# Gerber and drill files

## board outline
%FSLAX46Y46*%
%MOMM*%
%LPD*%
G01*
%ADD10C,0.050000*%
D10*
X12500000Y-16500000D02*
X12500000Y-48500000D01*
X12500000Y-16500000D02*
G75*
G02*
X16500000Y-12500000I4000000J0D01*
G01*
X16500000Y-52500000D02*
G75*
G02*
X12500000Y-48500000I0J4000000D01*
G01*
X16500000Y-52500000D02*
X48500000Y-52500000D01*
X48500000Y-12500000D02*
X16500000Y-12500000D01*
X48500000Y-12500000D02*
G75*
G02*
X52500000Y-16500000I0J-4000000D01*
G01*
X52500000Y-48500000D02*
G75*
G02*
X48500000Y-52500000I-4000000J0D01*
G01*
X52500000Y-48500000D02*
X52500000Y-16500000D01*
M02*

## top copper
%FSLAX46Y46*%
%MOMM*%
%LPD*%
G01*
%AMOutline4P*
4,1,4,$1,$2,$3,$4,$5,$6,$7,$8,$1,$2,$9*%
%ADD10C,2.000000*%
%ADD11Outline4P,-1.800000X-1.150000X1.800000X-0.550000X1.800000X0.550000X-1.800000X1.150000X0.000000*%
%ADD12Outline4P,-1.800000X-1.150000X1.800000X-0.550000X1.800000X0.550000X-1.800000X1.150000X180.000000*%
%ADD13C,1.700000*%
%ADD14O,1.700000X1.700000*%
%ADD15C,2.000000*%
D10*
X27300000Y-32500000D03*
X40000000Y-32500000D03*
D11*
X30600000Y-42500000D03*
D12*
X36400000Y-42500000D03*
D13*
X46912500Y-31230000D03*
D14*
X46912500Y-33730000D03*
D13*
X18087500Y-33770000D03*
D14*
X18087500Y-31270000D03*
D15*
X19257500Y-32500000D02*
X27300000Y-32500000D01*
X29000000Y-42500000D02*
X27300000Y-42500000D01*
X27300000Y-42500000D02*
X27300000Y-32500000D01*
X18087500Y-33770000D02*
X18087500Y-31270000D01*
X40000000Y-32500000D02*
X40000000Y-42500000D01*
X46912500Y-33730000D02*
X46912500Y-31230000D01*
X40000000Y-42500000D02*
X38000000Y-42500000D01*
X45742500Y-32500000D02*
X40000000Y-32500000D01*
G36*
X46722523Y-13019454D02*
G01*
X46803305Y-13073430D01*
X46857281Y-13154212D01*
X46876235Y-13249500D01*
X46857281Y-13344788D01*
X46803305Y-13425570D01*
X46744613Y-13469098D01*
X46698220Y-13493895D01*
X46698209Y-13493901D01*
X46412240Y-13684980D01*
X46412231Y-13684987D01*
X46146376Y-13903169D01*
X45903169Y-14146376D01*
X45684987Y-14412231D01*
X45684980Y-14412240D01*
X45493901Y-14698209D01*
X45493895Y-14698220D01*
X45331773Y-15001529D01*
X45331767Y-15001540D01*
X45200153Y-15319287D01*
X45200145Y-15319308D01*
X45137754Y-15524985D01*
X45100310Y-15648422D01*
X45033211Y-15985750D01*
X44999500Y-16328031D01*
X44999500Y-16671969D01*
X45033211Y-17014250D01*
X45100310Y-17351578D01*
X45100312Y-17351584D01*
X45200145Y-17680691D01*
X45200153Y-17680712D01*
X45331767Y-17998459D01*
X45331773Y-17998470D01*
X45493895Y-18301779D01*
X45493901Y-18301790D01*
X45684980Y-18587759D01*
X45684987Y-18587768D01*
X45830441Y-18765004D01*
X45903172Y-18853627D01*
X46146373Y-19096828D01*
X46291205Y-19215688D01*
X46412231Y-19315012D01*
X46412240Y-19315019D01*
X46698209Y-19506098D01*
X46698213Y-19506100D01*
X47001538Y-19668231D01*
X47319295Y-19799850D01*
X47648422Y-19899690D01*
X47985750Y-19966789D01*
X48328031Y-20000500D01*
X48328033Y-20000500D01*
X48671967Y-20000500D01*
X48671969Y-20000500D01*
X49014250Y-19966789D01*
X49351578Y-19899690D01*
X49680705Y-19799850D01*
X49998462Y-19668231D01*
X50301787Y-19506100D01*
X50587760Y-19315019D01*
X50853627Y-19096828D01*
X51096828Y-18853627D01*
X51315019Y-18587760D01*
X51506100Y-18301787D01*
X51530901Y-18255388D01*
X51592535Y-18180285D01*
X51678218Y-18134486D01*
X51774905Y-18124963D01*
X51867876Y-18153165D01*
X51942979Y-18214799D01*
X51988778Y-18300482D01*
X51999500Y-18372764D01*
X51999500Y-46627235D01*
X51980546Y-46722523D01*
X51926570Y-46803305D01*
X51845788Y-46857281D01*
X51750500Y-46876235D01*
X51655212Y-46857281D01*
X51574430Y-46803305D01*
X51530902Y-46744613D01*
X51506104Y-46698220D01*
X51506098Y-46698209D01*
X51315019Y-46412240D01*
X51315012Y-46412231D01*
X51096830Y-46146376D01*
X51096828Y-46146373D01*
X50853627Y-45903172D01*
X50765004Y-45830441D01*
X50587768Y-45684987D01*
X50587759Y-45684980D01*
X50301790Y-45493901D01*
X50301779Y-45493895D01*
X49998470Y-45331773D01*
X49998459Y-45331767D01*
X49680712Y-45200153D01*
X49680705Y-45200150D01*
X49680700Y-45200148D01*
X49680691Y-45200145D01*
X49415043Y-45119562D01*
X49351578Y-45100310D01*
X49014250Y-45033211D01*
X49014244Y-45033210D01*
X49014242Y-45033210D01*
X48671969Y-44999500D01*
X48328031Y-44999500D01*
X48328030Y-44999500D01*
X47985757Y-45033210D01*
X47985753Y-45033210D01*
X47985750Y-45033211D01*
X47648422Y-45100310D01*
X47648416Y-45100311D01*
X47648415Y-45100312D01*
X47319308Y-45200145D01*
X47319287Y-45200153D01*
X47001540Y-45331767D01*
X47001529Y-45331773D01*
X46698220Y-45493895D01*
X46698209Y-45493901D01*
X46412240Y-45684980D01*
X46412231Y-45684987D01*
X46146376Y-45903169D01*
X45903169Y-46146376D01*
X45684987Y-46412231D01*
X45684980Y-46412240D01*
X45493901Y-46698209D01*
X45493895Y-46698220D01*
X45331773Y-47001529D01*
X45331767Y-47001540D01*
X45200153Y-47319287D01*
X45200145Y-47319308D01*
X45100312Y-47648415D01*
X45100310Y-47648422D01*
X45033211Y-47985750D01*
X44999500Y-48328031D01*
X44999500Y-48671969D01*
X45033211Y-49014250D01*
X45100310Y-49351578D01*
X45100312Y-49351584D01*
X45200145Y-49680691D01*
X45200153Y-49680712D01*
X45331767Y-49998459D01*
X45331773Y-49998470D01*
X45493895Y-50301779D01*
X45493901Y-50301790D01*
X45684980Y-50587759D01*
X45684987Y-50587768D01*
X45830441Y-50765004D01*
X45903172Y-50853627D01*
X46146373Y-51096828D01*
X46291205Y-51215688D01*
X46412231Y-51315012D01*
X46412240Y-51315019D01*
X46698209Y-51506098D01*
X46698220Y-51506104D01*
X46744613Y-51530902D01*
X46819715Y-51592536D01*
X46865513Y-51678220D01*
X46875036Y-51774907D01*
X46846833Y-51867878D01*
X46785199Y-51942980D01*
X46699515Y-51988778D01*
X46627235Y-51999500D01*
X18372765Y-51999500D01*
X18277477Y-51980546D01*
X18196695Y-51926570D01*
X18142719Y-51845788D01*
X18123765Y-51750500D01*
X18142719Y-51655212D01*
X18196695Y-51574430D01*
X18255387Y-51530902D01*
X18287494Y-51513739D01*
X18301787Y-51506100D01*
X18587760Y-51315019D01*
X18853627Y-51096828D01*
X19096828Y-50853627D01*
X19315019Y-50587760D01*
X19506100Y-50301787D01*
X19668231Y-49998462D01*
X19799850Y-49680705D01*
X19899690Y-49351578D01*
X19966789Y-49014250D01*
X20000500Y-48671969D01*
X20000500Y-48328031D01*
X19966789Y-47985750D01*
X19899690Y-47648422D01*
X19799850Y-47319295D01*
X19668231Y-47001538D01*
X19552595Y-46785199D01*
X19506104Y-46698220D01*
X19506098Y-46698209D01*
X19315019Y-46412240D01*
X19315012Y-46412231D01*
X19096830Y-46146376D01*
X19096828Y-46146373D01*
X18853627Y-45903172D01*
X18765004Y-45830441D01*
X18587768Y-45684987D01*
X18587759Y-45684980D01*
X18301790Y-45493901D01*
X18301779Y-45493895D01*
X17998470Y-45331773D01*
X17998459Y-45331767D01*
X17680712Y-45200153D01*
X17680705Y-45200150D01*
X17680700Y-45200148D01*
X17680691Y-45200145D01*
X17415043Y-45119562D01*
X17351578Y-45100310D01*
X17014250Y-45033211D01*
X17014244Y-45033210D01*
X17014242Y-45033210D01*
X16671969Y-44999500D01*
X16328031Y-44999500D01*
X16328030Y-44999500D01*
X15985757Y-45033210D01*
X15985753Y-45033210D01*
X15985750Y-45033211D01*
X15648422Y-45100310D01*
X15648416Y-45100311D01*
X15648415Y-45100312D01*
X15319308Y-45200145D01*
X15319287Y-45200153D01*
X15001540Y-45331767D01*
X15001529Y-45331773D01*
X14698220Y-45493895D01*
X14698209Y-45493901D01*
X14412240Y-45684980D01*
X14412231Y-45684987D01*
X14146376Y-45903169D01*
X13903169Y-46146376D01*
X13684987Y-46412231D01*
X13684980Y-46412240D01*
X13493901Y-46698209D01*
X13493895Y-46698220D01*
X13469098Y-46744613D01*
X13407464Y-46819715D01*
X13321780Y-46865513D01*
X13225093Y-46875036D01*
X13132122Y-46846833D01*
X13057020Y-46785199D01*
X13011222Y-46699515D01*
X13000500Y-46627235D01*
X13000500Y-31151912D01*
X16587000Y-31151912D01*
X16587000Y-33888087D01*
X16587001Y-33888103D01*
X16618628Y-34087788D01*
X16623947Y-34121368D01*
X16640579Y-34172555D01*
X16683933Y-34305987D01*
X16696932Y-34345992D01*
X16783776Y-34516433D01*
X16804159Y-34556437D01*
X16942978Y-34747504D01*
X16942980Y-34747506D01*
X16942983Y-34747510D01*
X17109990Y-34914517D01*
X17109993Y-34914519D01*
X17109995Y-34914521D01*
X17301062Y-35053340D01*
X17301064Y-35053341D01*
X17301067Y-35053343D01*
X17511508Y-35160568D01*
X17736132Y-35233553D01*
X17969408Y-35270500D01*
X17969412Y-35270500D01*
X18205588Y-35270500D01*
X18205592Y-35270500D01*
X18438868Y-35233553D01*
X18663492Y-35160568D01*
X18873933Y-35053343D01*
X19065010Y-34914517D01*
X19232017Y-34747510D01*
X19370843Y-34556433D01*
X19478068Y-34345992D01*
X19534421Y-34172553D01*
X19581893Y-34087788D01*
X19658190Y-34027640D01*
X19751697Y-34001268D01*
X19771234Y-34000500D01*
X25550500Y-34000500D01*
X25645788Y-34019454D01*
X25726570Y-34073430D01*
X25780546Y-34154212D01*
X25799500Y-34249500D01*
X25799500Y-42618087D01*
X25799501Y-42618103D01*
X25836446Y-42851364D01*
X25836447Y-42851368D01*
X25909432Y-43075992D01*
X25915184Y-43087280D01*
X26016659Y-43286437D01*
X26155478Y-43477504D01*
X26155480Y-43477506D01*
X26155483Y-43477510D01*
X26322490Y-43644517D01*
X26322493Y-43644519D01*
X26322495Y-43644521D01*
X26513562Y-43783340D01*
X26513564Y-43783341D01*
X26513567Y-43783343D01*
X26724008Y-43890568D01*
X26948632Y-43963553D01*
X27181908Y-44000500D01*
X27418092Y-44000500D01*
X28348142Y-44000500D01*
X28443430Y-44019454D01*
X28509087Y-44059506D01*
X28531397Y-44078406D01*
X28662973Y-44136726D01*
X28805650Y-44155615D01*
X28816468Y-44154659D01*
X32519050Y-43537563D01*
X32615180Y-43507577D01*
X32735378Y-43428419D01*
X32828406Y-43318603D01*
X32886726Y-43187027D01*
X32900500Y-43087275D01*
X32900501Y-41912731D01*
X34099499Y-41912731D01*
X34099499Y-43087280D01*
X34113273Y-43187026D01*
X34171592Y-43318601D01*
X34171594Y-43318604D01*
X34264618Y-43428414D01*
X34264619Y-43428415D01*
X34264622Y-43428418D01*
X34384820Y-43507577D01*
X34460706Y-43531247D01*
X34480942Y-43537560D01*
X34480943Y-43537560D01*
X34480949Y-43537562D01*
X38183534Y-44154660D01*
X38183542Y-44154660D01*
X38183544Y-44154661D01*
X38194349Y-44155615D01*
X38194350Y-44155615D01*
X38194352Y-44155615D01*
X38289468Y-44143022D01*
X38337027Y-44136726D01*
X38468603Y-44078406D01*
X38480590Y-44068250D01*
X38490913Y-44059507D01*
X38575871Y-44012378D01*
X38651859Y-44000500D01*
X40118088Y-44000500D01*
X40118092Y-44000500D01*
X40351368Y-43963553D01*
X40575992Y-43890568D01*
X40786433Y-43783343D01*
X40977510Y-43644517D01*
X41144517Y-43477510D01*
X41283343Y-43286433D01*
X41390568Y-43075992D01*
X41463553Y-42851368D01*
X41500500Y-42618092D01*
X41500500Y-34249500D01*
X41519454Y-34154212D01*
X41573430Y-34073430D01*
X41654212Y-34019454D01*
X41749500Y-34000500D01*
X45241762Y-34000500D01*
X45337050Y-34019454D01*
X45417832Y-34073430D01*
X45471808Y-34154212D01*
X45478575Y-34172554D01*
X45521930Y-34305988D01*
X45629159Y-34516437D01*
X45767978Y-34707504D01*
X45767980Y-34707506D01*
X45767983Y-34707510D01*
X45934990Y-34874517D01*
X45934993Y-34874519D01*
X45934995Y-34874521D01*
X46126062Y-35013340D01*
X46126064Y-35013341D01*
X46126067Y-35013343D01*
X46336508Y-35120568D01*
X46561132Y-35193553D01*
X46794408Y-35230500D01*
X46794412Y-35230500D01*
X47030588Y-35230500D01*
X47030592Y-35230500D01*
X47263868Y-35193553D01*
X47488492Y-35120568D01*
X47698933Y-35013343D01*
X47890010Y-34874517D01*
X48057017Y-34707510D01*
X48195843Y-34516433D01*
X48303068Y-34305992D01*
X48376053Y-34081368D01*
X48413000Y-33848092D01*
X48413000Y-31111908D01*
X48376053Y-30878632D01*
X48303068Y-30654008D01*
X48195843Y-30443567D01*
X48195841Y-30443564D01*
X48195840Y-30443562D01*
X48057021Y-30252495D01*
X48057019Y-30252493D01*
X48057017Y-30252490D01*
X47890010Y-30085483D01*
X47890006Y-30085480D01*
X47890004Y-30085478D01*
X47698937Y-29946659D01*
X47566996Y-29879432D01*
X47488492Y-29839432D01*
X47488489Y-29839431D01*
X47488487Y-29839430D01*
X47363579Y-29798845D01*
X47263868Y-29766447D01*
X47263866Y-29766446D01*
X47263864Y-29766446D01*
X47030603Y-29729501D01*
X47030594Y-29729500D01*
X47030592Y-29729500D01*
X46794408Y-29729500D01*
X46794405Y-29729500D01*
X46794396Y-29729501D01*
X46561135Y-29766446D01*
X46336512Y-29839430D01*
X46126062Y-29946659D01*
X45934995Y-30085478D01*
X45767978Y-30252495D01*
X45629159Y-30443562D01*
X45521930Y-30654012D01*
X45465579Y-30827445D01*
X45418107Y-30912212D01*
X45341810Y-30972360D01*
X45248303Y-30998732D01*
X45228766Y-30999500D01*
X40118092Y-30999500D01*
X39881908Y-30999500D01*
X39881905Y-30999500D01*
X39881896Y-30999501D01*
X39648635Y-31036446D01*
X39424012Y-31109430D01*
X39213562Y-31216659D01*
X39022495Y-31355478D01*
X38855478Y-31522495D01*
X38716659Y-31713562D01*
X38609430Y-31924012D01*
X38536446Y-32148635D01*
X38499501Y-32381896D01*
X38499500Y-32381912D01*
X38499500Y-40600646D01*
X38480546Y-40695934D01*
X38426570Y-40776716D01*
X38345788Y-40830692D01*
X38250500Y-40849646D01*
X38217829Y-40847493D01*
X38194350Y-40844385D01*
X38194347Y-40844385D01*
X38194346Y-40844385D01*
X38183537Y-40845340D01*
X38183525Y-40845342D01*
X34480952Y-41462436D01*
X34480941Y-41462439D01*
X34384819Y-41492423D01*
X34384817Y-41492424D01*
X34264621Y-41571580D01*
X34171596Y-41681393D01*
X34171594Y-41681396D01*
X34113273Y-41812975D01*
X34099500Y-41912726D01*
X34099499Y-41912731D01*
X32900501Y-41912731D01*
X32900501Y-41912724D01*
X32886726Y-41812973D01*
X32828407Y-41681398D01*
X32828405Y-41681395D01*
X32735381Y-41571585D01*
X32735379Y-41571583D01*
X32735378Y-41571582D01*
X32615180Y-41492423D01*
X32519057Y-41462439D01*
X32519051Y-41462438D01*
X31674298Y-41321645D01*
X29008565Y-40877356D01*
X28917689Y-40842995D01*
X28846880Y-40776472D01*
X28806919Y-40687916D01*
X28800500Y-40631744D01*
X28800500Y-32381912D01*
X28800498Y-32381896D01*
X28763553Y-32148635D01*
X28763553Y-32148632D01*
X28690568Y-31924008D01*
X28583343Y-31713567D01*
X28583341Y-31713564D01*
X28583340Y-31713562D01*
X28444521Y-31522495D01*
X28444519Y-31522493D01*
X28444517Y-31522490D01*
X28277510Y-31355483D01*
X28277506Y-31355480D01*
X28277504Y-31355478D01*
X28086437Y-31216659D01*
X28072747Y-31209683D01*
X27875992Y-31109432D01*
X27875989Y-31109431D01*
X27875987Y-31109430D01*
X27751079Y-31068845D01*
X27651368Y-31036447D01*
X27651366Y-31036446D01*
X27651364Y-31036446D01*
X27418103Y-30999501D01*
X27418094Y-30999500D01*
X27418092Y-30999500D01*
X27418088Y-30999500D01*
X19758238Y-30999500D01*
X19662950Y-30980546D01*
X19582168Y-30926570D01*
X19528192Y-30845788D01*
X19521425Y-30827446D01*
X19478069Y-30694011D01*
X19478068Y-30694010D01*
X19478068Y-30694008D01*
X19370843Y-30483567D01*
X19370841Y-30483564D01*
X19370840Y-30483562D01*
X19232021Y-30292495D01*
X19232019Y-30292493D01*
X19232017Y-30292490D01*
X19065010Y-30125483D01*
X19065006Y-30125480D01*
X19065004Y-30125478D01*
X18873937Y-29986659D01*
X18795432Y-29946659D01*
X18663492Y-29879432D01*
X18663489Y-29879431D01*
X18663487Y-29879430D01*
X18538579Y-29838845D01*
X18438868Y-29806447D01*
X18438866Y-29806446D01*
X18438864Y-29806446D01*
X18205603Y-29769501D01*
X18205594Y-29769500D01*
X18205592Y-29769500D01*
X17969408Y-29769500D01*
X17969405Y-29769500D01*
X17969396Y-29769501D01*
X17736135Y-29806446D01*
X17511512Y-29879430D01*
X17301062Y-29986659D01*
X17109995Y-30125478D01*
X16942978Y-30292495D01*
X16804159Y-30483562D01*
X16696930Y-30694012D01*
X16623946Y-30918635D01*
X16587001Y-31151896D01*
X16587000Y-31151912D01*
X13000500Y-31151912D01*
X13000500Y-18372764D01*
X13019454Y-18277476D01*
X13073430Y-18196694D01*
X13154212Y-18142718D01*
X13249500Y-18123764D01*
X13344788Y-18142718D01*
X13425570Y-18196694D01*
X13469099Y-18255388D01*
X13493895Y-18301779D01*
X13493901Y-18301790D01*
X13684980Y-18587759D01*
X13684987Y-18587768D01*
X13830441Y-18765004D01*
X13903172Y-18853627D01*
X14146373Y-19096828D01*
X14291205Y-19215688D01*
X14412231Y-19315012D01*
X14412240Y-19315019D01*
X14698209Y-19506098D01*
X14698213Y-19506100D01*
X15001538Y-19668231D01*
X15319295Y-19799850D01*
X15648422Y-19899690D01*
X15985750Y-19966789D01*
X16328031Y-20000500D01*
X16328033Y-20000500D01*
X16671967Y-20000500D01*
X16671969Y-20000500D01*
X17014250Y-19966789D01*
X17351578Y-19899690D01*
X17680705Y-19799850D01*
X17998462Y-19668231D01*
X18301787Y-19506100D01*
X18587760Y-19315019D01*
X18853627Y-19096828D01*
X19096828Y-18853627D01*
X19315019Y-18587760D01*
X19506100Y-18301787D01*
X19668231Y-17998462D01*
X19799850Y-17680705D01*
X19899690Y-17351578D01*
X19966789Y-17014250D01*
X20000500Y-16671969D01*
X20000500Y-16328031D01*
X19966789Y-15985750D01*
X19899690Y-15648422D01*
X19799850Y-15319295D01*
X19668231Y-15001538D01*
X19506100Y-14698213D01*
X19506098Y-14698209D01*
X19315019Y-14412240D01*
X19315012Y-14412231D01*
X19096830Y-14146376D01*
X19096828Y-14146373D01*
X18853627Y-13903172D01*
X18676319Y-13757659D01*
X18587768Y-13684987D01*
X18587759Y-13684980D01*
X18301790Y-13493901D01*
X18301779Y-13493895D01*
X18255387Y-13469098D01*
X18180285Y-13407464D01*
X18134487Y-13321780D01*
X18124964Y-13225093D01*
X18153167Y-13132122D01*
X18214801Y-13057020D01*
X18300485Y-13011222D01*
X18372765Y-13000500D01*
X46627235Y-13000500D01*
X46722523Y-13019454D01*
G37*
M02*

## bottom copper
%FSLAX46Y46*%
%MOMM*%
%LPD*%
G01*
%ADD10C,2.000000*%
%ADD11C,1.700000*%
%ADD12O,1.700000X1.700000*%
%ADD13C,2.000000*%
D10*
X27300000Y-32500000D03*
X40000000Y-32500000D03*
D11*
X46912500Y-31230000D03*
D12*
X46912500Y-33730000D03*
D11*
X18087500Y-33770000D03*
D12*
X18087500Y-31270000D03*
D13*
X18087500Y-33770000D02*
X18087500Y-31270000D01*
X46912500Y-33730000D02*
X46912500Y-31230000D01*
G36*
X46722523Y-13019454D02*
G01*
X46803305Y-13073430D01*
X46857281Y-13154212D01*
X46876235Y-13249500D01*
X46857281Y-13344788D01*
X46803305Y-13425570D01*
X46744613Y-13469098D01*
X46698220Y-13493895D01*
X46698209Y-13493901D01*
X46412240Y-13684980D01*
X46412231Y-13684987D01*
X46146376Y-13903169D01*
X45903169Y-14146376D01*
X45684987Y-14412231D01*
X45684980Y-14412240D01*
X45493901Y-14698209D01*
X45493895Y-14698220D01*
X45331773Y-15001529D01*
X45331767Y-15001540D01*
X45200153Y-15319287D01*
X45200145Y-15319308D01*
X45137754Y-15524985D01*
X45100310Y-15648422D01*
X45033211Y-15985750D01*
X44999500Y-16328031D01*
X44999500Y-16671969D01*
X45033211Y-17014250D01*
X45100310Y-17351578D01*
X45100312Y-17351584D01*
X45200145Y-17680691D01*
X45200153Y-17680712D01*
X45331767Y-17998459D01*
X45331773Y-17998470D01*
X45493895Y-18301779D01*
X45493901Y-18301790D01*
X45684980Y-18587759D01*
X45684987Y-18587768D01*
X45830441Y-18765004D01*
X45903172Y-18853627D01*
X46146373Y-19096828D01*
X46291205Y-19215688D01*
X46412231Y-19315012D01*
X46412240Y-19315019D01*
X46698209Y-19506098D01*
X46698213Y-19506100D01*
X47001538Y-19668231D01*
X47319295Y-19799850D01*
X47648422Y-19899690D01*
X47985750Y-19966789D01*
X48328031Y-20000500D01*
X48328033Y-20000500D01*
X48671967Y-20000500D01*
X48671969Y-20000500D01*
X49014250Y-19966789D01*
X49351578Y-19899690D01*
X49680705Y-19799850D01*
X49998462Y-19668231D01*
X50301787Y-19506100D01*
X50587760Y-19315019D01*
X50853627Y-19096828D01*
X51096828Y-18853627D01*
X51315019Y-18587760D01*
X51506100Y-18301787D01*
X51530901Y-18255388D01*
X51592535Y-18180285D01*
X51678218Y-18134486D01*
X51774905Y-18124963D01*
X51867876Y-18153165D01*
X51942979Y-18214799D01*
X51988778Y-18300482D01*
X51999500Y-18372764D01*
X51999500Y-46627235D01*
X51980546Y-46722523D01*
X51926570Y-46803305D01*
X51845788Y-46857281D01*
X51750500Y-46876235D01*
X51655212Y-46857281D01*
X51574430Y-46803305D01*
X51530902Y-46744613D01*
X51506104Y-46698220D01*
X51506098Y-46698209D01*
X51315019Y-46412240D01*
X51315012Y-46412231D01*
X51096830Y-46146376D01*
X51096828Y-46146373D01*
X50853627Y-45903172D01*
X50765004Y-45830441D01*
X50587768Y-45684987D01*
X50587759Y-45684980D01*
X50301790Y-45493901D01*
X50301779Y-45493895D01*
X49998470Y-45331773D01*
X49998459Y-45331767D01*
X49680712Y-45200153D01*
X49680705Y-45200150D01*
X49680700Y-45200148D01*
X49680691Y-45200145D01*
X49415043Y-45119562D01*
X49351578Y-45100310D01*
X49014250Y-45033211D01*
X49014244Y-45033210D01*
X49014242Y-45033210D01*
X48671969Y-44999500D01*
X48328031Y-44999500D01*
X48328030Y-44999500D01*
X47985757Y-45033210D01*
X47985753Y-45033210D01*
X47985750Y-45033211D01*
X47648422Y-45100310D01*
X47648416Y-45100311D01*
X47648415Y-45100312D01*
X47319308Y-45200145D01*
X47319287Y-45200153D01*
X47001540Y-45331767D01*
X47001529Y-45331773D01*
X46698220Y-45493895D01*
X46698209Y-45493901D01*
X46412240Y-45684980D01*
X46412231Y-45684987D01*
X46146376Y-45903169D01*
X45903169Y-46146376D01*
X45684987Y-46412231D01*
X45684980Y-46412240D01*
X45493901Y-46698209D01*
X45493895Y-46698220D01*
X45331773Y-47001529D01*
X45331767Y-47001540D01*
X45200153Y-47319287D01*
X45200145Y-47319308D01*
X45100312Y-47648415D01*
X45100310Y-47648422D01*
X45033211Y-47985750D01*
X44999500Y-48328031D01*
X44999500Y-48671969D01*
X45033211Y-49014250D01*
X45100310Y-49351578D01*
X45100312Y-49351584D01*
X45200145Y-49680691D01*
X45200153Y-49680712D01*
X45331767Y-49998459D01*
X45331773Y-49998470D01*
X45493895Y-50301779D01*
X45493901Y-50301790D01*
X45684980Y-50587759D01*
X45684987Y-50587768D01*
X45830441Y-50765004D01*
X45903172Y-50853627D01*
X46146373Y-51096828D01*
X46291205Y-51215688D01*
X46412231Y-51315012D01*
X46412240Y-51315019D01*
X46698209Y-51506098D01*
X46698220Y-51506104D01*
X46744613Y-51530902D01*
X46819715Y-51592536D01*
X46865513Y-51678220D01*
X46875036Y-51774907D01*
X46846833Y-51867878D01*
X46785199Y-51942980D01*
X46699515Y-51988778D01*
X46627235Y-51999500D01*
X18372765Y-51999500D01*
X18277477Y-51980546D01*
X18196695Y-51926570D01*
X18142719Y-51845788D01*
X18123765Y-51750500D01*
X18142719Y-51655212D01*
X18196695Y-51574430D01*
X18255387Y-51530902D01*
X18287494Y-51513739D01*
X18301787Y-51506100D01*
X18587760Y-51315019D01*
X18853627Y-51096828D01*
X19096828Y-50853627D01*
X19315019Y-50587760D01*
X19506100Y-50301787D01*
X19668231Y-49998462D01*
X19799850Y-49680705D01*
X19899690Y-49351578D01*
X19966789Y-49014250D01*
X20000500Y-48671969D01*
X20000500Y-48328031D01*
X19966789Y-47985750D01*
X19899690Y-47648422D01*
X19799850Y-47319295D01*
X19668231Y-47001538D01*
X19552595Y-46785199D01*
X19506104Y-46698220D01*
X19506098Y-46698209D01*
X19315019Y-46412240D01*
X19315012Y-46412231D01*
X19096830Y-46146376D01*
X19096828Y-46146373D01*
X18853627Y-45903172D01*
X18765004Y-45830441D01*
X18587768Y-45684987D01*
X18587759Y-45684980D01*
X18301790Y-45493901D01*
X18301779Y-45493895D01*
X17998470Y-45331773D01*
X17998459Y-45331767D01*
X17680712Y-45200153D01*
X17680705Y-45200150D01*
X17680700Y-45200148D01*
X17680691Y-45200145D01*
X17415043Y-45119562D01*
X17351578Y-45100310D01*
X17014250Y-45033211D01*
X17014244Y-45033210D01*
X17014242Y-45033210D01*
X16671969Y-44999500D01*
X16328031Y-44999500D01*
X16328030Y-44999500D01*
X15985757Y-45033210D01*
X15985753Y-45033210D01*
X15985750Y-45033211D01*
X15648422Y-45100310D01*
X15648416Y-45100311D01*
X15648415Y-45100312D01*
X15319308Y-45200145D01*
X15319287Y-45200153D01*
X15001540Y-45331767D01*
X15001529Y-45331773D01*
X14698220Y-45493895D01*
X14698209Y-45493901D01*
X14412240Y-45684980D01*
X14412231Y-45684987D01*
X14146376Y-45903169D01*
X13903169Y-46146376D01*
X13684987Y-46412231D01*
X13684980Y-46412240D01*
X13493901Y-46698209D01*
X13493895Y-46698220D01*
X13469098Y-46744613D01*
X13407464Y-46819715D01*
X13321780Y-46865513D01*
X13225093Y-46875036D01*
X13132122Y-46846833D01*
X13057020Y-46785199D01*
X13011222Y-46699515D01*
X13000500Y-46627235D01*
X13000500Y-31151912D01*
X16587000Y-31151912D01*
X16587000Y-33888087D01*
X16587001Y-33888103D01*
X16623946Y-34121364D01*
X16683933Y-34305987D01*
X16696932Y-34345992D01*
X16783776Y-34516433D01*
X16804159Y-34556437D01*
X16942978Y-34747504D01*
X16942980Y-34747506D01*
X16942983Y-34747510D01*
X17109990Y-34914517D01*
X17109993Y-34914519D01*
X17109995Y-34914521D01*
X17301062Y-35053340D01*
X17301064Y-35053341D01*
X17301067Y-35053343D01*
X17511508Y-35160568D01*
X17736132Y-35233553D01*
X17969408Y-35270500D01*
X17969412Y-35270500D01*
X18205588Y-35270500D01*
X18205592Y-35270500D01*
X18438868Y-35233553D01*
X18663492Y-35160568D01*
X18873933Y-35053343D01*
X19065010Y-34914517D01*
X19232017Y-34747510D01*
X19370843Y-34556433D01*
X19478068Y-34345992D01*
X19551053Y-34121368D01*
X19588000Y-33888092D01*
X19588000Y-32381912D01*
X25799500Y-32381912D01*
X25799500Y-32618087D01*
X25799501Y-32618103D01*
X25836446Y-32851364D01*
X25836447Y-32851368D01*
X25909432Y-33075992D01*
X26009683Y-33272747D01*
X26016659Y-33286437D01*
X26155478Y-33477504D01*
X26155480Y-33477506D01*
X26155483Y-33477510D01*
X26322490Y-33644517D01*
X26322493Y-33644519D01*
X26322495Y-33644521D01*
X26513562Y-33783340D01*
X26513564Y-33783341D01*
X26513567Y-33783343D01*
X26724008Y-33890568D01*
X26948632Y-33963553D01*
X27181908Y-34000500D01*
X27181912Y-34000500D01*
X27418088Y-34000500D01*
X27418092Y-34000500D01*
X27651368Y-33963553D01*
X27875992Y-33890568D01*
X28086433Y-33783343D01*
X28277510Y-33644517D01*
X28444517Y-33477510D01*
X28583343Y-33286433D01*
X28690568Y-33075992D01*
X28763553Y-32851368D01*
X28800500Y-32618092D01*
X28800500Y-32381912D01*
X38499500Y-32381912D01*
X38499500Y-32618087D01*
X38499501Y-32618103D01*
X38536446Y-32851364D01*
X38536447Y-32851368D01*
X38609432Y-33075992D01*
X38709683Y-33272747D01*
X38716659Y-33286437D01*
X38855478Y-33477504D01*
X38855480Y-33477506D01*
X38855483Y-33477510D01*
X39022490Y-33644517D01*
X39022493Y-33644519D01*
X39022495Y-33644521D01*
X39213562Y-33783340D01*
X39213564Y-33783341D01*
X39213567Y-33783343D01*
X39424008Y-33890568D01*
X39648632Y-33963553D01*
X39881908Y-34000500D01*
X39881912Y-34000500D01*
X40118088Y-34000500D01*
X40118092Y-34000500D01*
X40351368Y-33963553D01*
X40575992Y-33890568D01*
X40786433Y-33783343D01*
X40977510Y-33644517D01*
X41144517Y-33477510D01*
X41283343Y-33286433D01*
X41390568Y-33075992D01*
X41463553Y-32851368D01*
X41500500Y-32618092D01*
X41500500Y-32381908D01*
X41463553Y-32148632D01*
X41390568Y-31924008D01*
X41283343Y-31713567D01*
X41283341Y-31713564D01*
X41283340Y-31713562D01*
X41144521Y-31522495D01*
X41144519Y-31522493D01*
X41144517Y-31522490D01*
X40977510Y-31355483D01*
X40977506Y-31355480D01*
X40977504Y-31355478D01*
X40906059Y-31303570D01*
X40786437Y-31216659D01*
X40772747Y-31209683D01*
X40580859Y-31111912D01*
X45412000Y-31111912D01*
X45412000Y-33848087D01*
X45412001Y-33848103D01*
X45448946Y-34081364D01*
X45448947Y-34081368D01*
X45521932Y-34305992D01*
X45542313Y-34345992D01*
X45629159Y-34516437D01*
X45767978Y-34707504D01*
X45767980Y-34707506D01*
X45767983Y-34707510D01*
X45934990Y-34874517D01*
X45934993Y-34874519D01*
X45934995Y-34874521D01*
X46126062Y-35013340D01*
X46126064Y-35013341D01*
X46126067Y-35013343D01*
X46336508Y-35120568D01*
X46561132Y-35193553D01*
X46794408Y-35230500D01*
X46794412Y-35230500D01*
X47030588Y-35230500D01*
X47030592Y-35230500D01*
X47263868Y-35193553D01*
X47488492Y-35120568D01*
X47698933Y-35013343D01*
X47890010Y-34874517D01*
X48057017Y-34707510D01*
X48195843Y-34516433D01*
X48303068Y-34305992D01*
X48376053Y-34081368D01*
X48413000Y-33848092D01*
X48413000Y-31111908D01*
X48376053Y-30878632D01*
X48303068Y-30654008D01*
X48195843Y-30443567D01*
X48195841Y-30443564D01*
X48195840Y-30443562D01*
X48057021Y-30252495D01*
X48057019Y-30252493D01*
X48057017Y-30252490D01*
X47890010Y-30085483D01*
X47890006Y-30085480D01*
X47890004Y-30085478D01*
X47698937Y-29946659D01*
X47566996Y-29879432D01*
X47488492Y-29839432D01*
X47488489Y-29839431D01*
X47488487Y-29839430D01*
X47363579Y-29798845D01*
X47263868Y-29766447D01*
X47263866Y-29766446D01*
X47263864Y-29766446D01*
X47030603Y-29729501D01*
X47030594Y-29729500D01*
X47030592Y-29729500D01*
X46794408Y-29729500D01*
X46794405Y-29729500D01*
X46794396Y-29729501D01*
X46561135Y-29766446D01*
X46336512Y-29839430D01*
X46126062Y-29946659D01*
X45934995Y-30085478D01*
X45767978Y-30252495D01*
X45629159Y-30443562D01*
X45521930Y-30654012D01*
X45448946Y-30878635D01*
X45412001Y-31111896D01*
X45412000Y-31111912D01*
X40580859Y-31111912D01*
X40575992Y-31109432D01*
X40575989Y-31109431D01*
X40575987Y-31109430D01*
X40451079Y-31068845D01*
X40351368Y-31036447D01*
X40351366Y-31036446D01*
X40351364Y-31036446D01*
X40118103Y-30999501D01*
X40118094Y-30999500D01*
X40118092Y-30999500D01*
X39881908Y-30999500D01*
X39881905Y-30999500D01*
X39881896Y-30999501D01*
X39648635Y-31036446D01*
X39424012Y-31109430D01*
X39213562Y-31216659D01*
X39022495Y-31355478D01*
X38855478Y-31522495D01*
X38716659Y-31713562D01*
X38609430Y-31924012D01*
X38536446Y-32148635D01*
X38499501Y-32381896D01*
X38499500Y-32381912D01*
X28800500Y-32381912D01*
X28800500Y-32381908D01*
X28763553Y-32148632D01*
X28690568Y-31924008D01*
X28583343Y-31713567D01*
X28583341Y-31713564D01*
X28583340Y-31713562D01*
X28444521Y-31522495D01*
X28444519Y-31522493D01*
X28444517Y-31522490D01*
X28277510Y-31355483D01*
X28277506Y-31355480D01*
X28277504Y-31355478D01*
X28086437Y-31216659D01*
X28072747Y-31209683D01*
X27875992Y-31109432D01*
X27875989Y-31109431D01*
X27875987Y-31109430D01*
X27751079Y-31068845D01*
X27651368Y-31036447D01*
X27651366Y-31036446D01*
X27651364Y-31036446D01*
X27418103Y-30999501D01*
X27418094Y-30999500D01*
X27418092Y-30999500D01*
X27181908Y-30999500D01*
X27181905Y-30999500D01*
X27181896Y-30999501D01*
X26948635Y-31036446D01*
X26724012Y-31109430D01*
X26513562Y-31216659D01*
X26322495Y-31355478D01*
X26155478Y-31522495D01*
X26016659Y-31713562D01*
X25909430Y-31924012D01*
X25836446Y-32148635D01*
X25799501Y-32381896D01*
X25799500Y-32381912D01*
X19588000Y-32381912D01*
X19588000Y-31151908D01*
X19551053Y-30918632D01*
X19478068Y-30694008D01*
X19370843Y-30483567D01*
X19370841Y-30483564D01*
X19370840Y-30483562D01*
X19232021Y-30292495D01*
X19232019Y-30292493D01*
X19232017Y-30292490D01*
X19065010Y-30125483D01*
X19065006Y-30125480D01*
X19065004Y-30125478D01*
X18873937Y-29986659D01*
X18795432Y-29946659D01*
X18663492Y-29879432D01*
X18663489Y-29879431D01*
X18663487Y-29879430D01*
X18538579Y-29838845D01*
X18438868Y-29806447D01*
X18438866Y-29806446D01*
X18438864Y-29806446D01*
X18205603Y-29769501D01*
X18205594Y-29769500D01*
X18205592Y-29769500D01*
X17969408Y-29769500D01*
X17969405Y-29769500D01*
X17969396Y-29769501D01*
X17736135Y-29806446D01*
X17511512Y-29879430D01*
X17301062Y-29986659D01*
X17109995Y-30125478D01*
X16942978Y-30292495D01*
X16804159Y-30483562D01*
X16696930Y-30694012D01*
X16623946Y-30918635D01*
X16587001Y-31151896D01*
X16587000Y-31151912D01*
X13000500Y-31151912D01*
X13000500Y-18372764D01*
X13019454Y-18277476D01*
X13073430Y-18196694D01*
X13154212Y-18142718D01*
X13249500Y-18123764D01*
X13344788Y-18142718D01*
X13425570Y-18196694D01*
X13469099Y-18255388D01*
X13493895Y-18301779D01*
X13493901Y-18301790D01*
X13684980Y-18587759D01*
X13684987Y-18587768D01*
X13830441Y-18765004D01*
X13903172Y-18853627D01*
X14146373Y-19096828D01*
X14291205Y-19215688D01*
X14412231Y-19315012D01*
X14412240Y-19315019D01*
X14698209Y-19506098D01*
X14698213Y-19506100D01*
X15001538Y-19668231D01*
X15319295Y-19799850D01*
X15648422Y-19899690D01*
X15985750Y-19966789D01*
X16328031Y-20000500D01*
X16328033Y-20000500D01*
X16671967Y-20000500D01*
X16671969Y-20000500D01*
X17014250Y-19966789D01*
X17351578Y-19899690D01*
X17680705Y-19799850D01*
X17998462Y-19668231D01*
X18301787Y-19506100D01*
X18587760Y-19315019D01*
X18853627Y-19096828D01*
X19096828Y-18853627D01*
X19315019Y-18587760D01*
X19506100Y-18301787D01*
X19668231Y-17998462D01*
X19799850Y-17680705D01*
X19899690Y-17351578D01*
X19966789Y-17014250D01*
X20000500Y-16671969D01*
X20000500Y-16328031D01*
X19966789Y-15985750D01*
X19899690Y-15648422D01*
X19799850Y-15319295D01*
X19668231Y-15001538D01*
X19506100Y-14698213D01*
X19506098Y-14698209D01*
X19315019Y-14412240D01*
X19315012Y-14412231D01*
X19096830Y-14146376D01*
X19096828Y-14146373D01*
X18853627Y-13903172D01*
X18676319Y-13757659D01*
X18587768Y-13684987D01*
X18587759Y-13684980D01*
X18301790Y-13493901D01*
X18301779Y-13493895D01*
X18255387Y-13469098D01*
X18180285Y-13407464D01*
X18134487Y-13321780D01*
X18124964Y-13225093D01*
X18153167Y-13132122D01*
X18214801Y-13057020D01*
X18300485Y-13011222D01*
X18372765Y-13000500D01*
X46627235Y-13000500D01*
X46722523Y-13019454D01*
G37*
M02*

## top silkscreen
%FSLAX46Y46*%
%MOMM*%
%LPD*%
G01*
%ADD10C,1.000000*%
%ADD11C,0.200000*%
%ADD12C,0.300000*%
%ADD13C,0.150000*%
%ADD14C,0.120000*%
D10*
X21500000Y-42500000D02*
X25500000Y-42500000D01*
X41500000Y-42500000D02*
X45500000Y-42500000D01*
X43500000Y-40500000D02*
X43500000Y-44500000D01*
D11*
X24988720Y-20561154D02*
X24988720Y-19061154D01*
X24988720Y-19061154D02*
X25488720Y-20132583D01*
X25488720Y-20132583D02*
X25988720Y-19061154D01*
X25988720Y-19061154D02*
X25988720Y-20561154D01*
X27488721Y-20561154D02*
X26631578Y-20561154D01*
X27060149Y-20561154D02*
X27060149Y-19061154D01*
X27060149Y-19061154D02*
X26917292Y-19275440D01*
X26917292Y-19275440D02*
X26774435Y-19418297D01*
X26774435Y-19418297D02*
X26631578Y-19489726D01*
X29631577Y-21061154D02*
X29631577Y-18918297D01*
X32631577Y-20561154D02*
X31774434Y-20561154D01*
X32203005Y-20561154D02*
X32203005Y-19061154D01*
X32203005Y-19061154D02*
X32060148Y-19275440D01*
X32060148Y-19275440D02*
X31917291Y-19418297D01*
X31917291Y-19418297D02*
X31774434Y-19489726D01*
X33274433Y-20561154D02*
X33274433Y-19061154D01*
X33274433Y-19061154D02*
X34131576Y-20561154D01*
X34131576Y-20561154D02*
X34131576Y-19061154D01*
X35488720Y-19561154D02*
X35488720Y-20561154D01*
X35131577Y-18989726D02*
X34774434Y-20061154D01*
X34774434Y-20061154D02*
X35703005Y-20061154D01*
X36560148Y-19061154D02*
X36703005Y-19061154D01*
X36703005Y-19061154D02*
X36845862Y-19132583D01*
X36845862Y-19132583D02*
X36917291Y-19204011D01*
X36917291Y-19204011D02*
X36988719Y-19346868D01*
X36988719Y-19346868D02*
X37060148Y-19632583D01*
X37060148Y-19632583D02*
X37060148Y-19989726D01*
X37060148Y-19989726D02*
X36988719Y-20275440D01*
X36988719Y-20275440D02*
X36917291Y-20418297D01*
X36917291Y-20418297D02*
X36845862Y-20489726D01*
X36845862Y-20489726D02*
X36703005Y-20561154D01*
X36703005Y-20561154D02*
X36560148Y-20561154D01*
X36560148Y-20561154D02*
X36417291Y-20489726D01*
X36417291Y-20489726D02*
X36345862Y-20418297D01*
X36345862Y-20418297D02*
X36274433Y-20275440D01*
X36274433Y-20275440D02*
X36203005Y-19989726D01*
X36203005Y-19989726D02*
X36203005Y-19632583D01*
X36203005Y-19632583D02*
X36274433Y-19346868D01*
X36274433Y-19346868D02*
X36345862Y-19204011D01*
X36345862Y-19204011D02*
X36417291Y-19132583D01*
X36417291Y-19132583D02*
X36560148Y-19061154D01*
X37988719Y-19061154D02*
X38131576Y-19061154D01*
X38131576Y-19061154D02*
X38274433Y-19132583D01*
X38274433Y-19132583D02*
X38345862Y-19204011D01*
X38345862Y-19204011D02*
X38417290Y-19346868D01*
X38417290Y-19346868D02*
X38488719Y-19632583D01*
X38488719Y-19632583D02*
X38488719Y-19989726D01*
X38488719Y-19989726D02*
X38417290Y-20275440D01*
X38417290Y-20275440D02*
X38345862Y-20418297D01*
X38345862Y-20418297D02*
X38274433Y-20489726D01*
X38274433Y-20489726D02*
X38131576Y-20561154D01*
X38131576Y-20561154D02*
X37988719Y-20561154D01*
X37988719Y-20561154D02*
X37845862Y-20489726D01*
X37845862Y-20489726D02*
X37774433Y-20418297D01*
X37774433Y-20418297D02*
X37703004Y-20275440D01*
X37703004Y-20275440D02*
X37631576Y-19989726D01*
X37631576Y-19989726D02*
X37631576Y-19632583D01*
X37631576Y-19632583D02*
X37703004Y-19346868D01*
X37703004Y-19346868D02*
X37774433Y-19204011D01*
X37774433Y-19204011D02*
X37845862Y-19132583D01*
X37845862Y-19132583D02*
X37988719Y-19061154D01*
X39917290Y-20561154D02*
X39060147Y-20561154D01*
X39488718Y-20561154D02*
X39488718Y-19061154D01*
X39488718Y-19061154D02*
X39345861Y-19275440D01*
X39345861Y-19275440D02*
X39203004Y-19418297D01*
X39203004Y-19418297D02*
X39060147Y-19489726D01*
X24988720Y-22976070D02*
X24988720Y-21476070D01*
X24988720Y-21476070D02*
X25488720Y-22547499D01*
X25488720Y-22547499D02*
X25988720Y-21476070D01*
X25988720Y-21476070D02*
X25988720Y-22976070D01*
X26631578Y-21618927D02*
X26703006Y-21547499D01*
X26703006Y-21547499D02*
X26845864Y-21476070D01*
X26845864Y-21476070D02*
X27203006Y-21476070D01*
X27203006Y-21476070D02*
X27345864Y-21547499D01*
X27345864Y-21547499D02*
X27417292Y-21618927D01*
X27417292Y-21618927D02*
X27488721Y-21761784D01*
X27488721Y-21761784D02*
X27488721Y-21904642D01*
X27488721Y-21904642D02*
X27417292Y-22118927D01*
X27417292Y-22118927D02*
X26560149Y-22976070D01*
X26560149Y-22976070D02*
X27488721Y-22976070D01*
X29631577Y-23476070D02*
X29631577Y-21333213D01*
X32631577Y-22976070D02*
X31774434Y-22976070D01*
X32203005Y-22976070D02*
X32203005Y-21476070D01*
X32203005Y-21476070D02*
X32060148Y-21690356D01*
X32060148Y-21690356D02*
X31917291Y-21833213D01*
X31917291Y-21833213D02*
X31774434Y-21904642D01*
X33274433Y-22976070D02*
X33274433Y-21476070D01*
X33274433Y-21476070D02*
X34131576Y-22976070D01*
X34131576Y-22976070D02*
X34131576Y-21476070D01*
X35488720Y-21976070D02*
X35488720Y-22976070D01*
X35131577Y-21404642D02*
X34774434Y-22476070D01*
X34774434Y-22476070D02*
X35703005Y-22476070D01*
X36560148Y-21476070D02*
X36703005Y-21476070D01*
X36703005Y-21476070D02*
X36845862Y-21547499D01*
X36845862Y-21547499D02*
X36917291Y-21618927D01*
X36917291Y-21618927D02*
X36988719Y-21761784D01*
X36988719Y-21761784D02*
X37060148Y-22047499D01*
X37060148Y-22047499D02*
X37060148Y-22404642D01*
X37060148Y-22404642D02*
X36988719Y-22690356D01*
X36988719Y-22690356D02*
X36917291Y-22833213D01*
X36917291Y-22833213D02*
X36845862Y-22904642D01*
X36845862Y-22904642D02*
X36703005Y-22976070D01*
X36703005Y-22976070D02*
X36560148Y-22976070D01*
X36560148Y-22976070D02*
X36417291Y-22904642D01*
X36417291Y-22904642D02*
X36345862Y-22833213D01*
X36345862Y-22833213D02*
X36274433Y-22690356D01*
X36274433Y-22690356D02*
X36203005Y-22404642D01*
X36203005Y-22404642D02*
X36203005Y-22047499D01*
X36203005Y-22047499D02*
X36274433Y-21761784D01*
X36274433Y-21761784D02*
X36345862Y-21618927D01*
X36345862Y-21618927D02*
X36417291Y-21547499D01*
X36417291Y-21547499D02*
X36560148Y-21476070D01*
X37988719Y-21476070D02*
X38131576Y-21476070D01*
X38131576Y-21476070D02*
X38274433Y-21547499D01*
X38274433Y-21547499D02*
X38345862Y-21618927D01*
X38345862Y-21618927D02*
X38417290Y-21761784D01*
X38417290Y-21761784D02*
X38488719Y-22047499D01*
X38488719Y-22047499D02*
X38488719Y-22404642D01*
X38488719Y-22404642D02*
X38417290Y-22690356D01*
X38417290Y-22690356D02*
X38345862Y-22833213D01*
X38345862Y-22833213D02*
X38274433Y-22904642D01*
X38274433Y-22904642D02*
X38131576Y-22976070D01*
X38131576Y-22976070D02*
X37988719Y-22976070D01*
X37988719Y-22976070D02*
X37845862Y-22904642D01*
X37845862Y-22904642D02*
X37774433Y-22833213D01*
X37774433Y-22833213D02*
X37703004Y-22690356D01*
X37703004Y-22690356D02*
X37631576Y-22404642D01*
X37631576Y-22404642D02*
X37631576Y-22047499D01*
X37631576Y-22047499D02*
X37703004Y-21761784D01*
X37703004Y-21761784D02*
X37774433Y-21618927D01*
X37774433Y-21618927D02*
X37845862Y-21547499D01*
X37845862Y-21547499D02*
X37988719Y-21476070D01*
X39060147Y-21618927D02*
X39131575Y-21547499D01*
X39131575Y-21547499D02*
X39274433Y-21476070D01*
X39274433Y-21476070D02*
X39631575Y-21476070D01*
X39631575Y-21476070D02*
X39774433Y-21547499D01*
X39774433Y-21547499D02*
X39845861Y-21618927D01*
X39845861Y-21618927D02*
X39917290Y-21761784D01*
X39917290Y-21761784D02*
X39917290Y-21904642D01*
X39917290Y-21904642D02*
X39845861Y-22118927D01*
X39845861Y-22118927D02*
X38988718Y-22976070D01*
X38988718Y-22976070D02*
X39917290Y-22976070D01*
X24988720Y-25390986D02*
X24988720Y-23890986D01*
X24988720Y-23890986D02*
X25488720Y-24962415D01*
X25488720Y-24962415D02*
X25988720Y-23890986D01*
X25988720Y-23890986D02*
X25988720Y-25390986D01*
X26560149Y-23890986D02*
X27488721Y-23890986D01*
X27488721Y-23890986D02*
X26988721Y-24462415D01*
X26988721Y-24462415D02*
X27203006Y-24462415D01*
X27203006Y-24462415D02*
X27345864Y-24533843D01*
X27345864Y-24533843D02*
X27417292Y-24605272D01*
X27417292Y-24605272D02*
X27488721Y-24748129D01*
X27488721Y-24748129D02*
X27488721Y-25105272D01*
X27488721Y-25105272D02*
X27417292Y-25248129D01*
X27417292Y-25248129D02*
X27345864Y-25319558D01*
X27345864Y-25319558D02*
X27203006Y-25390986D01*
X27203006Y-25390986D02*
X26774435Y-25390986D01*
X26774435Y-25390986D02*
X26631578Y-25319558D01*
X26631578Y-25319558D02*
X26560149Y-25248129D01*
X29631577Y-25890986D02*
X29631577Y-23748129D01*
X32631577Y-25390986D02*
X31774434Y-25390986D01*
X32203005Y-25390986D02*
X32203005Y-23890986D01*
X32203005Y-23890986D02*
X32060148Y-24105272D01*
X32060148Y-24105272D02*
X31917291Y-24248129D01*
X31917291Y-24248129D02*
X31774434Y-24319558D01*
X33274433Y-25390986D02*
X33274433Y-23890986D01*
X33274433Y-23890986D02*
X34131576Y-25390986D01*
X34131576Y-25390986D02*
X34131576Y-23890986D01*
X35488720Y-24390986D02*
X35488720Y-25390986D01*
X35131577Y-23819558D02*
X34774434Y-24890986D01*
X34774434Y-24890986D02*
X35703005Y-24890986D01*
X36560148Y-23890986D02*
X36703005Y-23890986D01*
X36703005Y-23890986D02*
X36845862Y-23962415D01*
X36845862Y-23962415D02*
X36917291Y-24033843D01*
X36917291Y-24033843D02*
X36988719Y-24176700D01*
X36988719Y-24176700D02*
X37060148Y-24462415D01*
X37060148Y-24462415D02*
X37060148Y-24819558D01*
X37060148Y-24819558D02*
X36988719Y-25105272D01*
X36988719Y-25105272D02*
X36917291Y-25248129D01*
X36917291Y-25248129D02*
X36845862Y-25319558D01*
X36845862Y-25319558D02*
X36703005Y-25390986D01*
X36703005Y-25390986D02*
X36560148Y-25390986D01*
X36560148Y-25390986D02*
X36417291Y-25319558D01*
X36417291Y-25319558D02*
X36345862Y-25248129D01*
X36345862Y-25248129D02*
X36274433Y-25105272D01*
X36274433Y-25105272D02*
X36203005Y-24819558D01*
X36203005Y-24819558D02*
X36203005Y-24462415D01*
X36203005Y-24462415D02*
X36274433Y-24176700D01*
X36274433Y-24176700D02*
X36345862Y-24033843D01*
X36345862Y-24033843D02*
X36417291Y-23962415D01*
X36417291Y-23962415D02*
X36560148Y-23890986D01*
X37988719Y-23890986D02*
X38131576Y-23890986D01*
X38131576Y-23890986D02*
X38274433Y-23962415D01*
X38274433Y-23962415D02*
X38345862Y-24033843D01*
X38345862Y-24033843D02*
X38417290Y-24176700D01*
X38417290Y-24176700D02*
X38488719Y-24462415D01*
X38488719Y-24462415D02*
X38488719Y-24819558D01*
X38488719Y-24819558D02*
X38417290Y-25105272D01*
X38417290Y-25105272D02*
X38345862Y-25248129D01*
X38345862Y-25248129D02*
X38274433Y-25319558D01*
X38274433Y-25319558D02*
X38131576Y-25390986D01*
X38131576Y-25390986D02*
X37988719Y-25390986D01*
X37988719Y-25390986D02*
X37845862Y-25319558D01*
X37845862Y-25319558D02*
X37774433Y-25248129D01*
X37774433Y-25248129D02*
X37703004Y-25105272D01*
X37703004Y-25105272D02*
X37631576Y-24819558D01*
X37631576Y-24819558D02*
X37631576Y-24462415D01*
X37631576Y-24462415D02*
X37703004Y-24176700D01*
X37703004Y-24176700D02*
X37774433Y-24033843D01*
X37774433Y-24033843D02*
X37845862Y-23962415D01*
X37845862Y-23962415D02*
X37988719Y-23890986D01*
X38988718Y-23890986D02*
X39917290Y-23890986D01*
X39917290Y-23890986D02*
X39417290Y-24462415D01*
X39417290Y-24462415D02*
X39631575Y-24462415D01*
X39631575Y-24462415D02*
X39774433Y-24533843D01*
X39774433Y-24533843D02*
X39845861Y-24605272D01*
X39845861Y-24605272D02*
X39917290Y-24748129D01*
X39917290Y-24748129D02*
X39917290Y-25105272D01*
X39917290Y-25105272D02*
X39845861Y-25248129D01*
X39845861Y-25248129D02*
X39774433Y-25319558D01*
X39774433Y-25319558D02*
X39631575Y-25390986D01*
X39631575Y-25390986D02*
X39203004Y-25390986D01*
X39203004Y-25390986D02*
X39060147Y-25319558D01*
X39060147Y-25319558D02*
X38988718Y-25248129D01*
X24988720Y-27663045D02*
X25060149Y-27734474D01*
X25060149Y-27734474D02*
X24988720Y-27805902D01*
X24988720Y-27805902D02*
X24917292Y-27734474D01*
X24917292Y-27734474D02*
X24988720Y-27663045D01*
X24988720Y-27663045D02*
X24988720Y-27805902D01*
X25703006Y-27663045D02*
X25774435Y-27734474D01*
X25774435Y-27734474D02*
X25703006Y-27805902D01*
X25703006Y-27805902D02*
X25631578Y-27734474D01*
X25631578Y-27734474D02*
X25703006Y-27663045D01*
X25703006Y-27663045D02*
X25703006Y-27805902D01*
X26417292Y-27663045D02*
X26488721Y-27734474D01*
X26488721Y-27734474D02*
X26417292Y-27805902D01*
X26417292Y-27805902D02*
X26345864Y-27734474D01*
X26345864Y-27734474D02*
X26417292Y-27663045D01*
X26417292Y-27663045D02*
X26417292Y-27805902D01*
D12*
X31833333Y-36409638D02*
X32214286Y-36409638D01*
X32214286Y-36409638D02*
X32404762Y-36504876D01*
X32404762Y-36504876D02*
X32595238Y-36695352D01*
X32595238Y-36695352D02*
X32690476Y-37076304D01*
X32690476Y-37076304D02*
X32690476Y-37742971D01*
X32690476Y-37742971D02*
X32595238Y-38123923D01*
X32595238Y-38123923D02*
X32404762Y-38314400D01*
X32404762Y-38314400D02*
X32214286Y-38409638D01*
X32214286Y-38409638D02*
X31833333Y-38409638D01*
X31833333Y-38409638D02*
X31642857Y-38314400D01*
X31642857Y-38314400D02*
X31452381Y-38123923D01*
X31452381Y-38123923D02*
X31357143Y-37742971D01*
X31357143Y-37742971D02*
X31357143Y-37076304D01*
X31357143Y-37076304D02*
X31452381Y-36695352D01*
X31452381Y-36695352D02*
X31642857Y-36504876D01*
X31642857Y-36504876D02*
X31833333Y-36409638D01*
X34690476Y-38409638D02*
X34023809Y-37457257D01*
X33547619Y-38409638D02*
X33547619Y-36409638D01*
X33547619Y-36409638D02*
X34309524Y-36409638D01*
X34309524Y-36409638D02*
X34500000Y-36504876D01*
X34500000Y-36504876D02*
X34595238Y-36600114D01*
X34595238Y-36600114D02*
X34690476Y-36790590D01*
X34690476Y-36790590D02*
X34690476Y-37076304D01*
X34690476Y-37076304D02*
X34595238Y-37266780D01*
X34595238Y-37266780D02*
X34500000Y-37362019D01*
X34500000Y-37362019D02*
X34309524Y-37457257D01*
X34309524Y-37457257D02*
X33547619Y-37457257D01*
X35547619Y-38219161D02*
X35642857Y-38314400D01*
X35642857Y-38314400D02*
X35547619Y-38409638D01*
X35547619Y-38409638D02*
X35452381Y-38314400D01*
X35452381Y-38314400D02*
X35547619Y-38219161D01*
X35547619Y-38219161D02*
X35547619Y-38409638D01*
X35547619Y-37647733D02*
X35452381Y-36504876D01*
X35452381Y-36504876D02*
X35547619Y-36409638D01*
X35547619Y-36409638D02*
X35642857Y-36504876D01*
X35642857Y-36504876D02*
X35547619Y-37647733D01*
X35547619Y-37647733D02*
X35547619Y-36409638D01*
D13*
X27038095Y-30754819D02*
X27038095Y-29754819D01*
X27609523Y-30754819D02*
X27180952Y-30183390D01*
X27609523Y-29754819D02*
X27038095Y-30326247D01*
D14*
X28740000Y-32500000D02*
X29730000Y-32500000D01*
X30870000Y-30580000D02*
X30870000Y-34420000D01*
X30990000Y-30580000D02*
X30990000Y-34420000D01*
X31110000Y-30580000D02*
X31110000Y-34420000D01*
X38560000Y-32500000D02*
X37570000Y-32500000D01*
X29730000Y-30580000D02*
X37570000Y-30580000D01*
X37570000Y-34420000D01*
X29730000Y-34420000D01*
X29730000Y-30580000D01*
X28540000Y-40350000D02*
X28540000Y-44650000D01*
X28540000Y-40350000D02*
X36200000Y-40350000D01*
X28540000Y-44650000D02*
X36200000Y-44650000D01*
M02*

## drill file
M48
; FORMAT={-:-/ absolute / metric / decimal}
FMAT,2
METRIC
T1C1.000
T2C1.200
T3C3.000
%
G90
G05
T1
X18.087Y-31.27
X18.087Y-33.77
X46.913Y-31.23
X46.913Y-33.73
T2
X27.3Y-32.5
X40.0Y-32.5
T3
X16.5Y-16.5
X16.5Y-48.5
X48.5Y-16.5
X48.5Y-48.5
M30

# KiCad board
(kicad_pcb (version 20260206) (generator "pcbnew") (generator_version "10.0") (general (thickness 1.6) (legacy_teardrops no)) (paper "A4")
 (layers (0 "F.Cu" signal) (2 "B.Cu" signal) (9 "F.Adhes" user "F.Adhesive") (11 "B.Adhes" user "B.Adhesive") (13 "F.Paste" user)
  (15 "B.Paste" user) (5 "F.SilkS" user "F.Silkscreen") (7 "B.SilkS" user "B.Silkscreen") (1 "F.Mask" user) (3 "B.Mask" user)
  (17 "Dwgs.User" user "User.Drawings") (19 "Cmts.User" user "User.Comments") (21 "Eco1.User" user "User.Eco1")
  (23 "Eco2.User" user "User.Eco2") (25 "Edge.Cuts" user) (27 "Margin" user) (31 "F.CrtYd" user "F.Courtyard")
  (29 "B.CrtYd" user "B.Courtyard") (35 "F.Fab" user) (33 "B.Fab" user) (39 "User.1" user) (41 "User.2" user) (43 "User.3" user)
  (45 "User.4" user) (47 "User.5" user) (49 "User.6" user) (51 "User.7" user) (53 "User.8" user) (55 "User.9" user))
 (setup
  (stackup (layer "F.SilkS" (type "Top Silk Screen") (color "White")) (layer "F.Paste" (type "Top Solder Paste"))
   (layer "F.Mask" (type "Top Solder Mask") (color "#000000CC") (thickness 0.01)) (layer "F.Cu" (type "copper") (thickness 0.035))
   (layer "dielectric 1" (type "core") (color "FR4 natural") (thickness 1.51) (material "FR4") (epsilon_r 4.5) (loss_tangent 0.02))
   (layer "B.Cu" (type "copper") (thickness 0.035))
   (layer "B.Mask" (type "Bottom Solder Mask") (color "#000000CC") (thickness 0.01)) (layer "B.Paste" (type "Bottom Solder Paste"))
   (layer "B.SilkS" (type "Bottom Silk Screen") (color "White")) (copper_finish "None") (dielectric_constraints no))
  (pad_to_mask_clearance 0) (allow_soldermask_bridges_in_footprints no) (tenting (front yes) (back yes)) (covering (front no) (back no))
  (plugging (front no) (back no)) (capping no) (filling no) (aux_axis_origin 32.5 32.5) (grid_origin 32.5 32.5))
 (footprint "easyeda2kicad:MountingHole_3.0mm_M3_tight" (layer "F.Cu") (at 16.5 16.5 90)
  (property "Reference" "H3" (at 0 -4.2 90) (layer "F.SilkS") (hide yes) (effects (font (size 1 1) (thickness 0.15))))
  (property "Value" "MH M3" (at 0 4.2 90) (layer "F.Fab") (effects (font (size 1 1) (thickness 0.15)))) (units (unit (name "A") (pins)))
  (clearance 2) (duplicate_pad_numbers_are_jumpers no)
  (pad "" np_thru_hole circle (at 0 0 90) (size 3 3) (drill 3) (layers "*.Cu" "*.Mask")))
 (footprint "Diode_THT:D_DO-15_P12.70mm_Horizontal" (layer "F.Cu") (at 27.3 32.5)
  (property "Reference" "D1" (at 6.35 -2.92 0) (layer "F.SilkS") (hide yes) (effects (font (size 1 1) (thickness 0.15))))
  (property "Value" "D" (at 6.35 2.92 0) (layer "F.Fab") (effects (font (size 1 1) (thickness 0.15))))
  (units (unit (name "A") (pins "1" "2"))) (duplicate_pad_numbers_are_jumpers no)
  (fp_line (start 1.44 0) (end 2.43 0) (stroke (width 0.12) (type solid)) (layer "F.SilkS"))
  (fp_line (start 3.57 -1.92) (end 3.57 1.92) (stroke (width 0.12) (type solid)) (layer "F.SilkS"))
  (fp_line (start 3.69 -1.92) (end 3.69 1.92) (stroke (width 0.12) (type solid)) (layer "F.SilkS"))
  (fp_line (start 3.81 -1.92) (end 3.81 1.92) (stroke (width 0.12) (type solid)) (layer "F.SilkS"))
  (fp_line (start 11.26 0) (end 10.27 0) (stroke (width 0.12) (type solid)) (layer "F.SilkS"))
  (fp_rect (start 2.43 -1.92) (end 10.27 1.92) (stroke (width 0.12) (type solid)) (fill no) (layer "F.SilkS"))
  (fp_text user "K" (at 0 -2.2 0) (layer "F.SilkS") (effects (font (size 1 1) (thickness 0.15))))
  (pad "1" thru_hole circle (at 0 0) (size 2 2) (drill 1.2) (layers "*.Cu" "*.Mask") (remove_unused_layers no) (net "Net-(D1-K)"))
  (pad "2" thru_hole circle (at 12.7 0) (size 2 2) (drill 1.2) (layers "*.Cu" "*.Mask") (remove_unused_layers no) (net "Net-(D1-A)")))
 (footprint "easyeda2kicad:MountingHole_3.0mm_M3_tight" (layer "F.Cu") (at 16.5 48.5 90)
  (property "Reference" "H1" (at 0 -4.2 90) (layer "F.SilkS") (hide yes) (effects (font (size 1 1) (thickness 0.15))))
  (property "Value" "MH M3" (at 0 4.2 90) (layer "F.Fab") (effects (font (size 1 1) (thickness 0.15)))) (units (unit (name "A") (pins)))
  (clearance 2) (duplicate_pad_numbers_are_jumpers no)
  (pad "" np_thru_hole circle (at 0 0 90) (size 3 3) (drill 3) (layers "*.Cu" "*.Mask")))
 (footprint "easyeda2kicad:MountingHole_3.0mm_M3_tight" (layer "F.Cu") (at 48.5 16.5 90)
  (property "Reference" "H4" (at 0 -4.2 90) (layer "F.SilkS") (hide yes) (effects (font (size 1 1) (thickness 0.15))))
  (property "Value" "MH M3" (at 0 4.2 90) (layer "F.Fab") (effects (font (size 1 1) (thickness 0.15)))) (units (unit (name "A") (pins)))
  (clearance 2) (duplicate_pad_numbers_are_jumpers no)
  (pad "" np_thru_hole circle (at 0 0 90) (size 3 3) (drill 3) (layers "*.Cu" "*.Mask")))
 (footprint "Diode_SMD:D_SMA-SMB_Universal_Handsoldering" (layer "F.Cu") (at 33.5 42.5)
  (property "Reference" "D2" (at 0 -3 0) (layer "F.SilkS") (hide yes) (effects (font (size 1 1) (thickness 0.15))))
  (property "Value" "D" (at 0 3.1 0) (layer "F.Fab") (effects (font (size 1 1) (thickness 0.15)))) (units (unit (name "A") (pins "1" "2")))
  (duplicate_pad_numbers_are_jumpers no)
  (fp_line (start -4.96 -2.15) (end -4.96 2.15) (stroke (width 0.12) (type solid)) (layer "F.SilkS"))
  (fp_line (start -4.96 -2.15) (end 2.7 -2.15) (stroke (width 0.12) (type solid)) (layer "F.SilkS"))
  (fp_line (start -4.96 2.15) (end 2.7 2.15) (stroke (width 0.12) (type solid)) (layer "F.SilkS"))
  (pad "1" smd trapezoid (at -2.9 0) (size 3.6 1.7) (rect_delta 0.6 0) (layers "F.Cu" "F.Mask" "F.Paste") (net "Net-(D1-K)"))
  (pad "2" smd trapezoid (at 2.9 0 180) (size 3.6 1.7) (rect_delta 0.6 0) (layers "F.Cu" "F.Mask" "F.Paste") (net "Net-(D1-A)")))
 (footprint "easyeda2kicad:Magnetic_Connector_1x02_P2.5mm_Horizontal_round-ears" (layer "F.Cu") (at 47.0125 32.5)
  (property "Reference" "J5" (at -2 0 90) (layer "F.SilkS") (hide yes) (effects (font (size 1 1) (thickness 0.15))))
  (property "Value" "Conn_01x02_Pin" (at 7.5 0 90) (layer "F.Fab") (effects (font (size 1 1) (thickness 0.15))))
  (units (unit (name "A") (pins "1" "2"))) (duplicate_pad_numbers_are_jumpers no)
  (pad "1" thru_hole circle (at -0.1 -1.27) (size 1.7 1.7) (drill 1) (layers "*.Cu" "*.Mask") (remove_unused_layers no) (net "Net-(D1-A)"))
  (pad "2" thru_hole oval (at -0.1 1.23) (size 1.7 1.7) (drill 1) (layers "*.Cu" "*.Mask") (remove_unused_layers no) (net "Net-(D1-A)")))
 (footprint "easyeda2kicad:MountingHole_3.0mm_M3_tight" (layer "F.Cu") (at 48.5 48.5 90)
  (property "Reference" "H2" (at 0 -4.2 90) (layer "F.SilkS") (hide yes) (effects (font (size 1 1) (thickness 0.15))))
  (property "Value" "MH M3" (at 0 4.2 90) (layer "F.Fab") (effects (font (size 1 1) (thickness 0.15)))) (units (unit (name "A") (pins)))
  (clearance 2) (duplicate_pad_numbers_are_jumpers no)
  (pad "" np_thru_hole circle (at 0 0 90) (size 3 3) (drill 3) (layers "*.Cu" "*.Mask")))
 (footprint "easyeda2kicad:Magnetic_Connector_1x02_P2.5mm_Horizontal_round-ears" (layer "F.Cu") (at 17.9875 32.5 180)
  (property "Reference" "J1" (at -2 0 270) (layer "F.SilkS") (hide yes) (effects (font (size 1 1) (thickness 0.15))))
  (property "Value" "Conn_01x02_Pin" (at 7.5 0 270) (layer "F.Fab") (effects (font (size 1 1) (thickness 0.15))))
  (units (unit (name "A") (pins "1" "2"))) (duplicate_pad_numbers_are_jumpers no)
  (pad "1" thru_hole circle (at -0.1 -1.27 180) (size 1.7 1.7) (drill 1) (layers "*.Cu" "*.Mask") (remove_unused_layers no)
   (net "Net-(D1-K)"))
  (pad "2" thru_hole oval (at -0.1 1.23 180) (size 1.7 1.7) (drill 1) (layers "*.Cu" "*.Mask") (remove_unused_layers no) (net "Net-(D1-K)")))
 (gr_line (start 21.5 42.5) (end 25.5 42.5) (stroke (width 1) (type default)) (layer "F.SilkS"))
 (gr_line (start 41.5 42.5) (end 45.5 42.5) (stroke (width 1) (type default)) (layer "F.SilkS"))
 (gr_line (start 43.5 40.5) (end 43.5 44.5) (stroke (width 1) (type default)) (layer "F.SilkS"))
 (gr_line (start 12.5 16.5) (end 12.5 48.5) (stroke (width 0.05) (type default)) (layer "Edge.Cuts"))
 (gr_arc (start 12.5 16.5) (mid 13.671573 13.671573) (end 16.5 12.5) (stroke (width 0.05) (type default)) (layer "Edge.Cuts"))
 (gr_arc (start 16.5 52.5) (mid 13.671573 51.328427) (end 12.5 48.5) (stroke (width 0.05) (type default)) (layer "Edge.Cuts"))
 (gr_line (start 16.5 52.5) (end 48.5 52.5) (stroke (width 0.05) (type default)) (layer "Edge.Cuts"))
 (gr_line (start 48.5 12.5) (end 16.5 12.5) (stroke (width 0.05) (type default)) (layer "Edge.Cuts"))
 (gr_arc (start 48.5 12.5) (mid 51.328427 13.671573) (end 52.5 16.5) (stroke (width 0.05) (type default)) (layer "Edge.Cuts"))
 (gr_arc (start 52.5 48.5) (mid 51.328427 51.328427) (end 48.5 52.5) (stroke (width 0.05) (type default)) (layer "Edge.Cuts"))
 (gr_line (start 52.5 48.5) (end 52.5 16.5) (stroke (width 0.05) (type default)) (layer "Edge.Cuts"))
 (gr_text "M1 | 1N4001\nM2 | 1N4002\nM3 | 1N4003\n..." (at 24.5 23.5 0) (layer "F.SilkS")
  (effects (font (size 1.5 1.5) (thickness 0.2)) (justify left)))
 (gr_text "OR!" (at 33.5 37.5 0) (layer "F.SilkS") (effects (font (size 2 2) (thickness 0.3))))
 (segment (start 19.2575 32.5) (end 27.3 32.5) (width 2) (layer "F.Cu") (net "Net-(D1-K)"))
 (segment (start 29 42.5) (end 27.3 42.5) (width 2) (layer "F.Cu") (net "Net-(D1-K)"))
 (segment (start 27.3 42.5) (end 27.3 32.5) (width 2) (layer "F.Cu") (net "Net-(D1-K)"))
 (segment (start 18.0875 33.77) (end 18.0875 31.27) (width 2) (layer "F.Cu") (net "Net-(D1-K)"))
 (segment (start 18.0875 33.77) (end 18.0875 31.27) (width 2) (layer "B.Cu") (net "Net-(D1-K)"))
 (segment (start 40 32.5) (end 40 42.5) (width 2) (layer "F.Cu") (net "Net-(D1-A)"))
 (segment (start 46.9125 33.73) (end 46.9125 31.23) (width 2) (layer "F.Cu") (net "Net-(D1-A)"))
 (segment (start 40 42.5) (end 38 42.5) (width 2) (layer "F.Cu") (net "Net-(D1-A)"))
 (segment (start 45.7425 32.5) (end 40 32.5) (width 2) (layer "F.Cu") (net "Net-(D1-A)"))
 (segment (start 46.9125 33.73) (end 46.9125 31.23) (width 2) (layer "B.Cu") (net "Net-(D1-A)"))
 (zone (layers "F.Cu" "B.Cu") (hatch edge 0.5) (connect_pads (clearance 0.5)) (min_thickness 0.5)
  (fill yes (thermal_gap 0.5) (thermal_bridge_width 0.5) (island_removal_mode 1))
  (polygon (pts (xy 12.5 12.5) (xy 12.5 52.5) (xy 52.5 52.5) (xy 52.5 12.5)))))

